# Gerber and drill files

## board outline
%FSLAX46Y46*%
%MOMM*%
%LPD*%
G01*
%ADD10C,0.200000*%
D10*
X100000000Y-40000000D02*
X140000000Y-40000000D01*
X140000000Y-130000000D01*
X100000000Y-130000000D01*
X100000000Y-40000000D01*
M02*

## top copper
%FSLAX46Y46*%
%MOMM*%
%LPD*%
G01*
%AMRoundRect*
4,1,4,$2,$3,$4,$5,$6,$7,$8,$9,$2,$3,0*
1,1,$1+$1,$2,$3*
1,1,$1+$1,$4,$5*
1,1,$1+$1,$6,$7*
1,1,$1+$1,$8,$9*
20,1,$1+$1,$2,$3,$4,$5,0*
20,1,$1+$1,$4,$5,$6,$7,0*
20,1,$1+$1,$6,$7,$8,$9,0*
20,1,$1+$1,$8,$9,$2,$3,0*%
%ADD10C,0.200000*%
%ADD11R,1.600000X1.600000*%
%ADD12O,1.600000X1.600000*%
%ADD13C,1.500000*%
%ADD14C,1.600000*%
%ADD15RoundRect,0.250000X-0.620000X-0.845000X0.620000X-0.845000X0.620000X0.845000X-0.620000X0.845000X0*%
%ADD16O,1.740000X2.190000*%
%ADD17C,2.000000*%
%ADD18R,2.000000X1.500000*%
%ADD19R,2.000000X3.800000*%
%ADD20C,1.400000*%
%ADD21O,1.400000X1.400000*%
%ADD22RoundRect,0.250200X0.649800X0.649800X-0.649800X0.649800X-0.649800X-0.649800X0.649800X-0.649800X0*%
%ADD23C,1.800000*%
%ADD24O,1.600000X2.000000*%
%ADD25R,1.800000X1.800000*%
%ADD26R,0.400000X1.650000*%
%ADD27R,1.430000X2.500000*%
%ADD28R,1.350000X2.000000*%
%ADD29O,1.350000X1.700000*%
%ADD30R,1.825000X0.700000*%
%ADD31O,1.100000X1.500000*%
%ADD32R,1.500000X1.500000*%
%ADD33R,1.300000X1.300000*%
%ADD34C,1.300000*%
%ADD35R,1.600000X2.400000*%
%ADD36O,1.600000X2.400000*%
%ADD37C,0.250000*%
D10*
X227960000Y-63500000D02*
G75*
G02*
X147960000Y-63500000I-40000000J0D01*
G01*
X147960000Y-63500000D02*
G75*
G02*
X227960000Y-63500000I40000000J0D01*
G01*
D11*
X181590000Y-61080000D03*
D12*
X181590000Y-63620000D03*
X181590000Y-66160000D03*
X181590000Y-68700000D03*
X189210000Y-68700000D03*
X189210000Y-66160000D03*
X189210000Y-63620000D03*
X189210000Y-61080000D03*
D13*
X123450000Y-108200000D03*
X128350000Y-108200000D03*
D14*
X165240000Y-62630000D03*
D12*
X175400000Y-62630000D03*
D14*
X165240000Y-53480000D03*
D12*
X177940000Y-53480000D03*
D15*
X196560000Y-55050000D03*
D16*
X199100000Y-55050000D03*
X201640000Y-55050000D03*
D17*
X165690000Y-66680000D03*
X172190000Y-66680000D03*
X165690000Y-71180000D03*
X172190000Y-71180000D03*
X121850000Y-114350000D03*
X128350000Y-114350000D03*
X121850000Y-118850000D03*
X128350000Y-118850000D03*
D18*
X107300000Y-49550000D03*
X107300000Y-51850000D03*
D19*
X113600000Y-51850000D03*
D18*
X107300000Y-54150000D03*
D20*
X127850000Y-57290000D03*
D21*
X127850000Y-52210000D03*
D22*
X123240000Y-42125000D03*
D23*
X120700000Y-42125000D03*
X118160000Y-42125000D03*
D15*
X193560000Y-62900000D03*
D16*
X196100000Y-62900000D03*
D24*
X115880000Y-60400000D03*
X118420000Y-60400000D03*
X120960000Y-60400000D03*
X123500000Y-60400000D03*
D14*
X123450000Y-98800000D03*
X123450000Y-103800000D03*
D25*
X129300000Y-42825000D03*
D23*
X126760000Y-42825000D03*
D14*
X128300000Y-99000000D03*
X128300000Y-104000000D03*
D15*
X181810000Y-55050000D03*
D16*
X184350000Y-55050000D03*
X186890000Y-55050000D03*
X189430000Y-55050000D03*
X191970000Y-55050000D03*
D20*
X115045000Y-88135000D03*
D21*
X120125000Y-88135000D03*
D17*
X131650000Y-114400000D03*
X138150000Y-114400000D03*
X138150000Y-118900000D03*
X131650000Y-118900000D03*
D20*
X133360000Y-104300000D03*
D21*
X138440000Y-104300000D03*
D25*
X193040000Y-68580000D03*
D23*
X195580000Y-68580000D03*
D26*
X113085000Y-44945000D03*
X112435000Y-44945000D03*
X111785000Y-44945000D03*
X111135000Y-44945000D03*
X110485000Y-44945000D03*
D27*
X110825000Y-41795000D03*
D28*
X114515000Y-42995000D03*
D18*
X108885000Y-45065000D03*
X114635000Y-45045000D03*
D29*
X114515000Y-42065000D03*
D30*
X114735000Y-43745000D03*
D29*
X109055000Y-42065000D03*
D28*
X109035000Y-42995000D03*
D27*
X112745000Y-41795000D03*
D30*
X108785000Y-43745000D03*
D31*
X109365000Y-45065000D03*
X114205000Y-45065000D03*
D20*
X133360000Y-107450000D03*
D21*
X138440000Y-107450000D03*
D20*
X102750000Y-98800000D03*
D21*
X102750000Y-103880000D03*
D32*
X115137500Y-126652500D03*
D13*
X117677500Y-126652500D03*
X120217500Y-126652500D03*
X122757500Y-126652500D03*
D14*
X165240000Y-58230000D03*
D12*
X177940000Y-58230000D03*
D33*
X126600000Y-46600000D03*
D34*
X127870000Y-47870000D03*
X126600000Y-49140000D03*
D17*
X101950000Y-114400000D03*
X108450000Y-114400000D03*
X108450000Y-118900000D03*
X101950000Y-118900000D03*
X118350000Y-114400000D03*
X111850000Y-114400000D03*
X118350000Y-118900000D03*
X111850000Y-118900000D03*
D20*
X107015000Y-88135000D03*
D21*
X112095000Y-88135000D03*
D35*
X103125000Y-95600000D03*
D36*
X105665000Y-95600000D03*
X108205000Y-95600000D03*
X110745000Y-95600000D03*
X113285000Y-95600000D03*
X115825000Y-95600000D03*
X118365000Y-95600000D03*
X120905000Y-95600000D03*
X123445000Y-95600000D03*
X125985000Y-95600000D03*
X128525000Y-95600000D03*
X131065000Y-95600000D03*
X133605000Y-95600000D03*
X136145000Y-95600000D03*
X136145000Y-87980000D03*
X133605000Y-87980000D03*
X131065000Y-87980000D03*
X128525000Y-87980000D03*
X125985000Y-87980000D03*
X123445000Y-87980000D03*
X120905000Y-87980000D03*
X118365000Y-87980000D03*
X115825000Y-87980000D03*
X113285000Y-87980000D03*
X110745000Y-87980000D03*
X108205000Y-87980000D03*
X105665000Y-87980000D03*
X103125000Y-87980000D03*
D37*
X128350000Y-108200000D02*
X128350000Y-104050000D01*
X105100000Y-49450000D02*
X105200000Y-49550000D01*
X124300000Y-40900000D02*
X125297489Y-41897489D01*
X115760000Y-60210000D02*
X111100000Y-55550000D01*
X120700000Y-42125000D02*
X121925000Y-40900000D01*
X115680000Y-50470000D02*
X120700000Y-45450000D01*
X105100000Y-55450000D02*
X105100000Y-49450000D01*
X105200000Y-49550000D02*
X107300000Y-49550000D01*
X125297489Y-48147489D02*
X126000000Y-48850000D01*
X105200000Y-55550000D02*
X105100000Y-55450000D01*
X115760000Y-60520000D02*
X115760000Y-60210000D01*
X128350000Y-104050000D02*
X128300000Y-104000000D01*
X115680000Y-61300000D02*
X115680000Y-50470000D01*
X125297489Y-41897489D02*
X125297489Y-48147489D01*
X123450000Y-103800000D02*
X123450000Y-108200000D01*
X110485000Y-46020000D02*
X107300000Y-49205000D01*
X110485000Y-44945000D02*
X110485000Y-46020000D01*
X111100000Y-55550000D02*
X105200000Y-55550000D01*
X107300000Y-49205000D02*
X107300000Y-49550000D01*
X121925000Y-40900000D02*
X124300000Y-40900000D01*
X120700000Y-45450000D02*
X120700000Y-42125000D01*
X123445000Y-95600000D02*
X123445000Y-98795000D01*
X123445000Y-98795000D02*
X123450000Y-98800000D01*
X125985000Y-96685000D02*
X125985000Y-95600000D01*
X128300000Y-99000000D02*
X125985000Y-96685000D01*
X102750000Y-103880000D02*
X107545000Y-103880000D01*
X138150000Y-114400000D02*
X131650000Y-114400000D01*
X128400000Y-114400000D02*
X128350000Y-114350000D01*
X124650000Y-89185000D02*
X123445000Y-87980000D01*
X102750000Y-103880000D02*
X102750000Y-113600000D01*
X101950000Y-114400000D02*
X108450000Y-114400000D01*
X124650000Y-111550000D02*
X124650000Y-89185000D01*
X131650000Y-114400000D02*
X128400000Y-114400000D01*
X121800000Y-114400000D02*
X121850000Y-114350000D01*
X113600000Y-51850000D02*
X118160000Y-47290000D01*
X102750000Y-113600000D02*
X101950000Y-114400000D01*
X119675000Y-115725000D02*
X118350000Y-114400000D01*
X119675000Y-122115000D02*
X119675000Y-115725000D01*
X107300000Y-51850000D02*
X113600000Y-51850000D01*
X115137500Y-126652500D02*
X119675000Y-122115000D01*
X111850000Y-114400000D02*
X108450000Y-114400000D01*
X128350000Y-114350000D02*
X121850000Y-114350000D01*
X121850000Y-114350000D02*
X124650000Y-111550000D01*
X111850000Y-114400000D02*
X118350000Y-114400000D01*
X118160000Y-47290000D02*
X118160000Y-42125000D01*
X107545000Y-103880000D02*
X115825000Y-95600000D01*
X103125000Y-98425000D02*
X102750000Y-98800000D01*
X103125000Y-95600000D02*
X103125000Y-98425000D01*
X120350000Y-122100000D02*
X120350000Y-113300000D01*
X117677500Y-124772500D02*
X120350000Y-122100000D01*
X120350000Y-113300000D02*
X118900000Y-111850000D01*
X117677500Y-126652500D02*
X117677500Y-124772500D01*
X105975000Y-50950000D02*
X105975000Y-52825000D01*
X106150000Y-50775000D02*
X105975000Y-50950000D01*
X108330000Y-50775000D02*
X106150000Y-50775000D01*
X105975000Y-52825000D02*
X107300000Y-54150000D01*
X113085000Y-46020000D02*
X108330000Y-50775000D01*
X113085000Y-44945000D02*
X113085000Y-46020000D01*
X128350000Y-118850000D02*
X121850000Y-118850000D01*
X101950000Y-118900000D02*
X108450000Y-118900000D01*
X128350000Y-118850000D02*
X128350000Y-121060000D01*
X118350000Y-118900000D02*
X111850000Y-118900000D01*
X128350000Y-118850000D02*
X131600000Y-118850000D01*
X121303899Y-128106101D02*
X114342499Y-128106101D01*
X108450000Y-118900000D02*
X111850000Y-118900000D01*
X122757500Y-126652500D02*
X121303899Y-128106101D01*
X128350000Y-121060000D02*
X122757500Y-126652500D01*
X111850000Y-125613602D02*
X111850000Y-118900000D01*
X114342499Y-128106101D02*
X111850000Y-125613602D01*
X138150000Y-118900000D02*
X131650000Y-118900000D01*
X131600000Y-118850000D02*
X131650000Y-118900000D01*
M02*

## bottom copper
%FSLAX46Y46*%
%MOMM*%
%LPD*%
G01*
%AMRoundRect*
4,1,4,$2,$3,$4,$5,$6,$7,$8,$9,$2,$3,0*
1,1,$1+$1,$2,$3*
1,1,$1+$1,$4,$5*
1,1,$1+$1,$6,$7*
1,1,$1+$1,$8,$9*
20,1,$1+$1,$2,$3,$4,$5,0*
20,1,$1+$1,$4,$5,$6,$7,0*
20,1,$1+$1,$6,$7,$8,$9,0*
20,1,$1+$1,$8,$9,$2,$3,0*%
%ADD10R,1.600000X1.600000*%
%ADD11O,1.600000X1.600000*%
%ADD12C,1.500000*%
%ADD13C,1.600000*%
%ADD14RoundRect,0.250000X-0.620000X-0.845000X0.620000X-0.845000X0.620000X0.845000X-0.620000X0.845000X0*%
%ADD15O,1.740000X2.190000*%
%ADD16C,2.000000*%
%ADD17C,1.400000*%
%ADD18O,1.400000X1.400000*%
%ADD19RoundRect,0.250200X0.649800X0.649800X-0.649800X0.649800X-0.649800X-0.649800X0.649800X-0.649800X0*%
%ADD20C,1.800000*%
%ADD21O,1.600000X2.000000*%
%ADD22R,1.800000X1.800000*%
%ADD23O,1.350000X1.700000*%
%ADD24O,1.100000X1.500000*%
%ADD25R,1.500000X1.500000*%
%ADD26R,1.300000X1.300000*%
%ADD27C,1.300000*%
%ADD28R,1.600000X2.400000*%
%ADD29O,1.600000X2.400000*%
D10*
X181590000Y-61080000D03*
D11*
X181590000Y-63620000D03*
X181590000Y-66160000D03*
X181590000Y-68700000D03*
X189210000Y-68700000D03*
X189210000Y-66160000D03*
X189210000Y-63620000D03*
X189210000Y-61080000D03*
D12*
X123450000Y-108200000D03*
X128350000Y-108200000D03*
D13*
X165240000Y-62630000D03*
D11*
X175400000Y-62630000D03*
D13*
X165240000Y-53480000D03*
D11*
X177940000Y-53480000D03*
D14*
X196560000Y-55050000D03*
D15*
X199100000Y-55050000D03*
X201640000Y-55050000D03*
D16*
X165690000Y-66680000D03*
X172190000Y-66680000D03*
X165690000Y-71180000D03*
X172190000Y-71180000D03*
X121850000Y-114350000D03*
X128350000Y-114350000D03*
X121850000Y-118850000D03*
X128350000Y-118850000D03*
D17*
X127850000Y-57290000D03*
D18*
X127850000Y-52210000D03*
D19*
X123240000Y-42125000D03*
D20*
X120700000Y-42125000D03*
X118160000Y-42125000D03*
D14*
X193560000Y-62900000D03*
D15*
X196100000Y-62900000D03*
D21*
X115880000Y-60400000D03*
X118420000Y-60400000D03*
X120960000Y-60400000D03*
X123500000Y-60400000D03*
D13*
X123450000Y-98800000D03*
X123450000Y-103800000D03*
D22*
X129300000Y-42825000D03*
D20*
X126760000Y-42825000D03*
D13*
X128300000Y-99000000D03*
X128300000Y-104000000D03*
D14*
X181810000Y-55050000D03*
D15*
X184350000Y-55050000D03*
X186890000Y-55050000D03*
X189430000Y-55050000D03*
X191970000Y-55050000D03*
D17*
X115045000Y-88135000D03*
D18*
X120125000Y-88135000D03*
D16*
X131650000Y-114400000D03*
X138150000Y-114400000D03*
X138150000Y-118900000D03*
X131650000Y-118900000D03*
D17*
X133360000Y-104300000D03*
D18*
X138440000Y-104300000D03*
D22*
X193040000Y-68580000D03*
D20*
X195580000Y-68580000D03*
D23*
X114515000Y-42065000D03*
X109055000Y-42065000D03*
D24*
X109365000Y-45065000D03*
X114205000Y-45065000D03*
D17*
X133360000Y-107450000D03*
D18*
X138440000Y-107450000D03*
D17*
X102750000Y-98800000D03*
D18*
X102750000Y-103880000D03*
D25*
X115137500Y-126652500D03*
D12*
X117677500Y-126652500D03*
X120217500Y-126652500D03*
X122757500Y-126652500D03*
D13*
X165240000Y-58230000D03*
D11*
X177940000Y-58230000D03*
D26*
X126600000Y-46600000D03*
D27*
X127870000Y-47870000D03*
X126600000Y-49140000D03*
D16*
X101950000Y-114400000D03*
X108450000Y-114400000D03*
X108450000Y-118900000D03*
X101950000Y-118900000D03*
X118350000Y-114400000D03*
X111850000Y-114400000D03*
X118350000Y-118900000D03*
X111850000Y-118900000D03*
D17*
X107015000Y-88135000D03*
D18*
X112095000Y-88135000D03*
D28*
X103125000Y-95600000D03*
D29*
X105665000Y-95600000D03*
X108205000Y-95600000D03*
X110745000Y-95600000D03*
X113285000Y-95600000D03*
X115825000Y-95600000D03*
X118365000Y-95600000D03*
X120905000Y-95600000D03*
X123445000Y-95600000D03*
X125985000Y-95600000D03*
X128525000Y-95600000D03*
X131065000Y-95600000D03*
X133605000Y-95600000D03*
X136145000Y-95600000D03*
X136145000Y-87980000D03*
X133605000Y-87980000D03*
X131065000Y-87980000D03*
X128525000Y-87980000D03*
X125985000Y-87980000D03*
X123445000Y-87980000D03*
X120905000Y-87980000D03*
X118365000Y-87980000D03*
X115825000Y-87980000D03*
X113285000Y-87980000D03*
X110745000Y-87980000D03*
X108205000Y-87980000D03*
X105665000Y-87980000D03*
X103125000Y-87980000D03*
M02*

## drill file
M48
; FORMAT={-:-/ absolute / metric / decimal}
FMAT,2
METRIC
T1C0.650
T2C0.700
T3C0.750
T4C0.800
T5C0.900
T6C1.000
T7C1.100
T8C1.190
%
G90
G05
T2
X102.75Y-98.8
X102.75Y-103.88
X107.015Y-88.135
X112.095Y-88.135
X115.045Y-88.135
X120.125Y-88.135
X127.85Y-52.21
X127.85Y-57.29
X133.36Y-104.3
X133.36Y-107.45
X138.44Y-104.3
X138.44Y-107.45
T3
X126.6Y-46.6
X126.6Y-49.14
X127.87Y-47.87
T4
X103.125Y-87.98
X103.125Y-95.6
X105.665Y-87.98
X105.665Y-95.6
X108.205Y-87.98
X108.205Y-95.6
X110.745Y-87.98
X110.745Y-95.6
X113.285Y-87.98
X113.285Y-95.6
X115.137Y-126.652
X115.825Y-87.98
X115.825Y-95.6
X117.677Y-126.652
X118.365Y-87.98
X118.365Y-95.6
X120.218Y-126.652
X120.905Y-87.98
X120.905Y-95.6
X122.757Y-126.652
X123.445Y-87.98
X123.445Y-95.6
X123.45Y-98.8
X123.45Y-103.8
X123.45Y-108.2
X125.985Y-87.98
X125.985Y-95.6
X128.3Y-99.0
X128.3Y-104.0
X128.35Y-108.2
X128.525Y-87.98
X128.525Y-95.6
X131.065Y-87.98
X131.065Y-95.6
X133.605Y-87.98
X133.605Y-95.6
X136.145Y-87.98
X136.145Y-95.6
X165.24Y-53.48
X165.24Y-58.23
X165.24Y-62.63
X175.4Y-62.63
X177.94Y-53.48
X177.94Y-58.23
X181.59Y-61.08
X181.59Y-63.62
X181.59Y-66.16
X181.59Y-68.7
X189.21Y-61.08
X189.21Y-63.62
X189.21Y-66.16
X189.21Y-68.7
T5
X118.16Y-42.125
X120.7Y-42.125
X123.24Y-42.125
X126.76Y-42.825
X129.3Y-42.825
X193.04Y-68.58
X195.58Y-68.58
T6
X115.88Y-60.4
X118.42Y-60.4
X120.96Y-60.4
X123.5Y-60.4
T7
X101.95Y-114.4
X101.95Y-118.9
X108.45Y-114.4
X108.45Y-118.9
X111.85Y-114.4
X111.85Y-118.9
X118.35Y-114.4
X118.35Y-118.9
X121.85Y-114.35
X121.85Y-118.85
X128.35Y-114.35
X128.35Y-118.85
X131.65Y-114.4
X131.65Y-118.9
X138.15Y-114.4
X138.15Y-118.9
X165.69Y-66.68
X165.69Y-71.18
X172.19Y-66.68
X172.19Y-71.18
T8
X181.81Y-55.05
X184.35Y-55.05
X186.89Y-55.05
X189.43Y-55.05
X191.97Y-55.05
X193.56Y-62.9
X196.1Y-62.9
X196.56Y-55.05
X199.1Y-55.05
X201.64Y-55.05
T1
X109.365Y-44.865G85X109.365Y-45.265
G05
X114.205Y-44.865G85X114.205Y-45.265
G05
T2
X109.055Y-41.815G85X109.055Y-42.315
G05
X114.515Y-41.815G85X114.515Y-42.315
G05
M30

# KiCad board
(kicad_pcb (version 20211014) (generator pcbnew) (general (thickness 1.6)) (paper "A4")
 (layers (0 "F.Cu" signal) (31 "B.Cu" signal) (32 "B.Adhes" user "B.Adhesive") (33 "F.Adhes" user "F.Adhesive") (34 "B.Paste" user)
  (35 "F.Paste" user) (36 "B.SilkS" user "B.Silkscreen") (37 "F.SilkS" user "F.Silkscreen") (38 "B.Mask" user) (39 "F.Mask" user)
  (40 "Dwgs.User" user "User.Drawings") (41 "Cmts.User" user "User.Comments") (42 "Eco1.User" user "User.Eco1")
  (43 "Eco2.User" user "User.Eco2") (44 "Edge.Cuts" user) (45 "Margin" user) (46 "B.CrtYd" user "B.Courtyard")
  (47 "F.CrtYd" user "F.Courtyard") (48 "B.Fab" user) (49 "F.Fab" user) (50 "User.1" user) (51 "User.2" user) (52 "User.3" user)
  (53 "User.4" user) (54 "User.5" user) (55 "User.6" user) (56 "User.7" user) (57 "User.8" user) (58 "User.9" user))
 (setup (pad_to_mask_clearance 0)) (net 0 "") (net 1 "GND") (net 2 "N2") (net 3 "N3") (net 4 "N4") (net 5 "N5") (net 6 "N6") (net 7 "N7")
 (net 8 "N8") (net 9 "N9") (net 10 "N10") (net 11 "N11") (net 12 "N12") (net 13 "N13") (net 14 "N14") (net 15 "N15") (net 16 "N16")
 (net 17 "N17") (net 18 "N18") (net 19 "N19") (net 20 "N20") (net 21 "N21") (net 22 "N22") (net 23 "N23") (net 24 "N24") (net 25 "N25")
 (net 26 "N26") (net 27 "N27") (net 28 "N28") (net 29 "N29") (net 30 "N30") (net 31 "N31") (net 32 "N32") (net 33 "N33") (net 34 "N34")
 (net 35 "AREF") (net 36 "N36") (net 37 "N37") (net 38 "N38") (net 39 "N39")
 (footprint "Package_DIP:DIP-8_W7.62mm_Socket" (layer "F.Cu") (at 181.59 61.08)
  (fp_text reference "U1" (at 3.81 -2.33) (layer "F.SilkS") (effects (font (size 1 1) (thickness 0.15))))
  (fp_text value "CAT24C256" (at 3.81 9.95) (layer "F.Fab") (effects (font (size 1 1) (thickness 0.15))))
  (pad "1" thru_hole rect (at 0 0) (size 1.6 1.6) (drill 0.8) (layers *.Cu *.Mask) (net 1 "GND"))
  (pad "2" thru_hole oval (at 0 2.54) (size 1.6 1.6) (drill 0.8) (layers *.Cu *.Mask) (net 1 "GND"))
  (pad "3" thru_hole oval (at 0 5.08) (size 1.6 1.6) (drill 0.8) (layers *.Cu *.Mask) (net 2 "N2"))
  (pad "4" thru_hole oval (at 0 7.62) (size 1.6 1.6) (drill 0.8) (layers *.Cu *.Mask) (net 1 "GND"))
  (pad "5" thru_hole oval (at 7.62 7.62) (size 1.6 1.6) (drill 0.8) (layers *.Cu *.Mask) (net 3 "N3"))
  (pad "6" thru_hole oval (at 7.62 5.08) (size 1.6 1.6) (drill 0.8) (layers *.Cu *.Mask) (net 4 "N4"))
  (pad "7" thru_hole oval (at 7.62 2.54) (size 1.6 1.6) (drill 0.8) (layers *.Cu *.Mask) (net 1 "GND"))
  (pad "8" thru_hole oval (at 7.62 0) (size 1.6 1.6) (drill 0.8) (layers *.Cu *.Mask) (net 2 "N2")))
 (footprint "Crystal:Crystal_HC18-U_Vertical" (layer "F.Cu") (at 123.45 108.2)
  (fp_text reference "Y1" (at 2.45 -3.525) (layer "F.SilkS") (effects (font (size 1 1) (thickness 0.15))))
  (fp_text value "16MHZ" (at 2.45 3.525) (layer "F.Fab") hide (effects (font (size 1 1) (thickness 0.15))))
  (pad "1" thru_hole circle (at 0 0) (size 1.5 1.5) (drill 0.8) (layers *.Cu *.Mask) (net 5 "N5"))
  (pad "2" thru_hole circle (at 4.9 0) (size 1.5 1.5) (drill 0.8) (layers *.Cu *.Mask) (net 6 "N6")))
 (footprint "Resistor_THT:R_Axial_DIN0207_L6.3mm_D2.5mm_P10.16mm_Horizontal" (layer "F.Cu") (at 165.24 62.63)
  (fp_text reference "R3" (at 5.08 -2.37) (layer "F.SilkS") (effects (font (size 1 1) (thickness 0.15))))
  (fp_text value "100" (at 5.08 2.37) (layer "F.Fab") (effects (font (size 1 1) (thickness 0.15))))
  (pad "1" thru_hole circle (at 0 0) (size 1.6 1.6) (drill 0.8) (layers *.Cu *.Mask) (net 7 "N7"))
  (pad "2" thru_hole oval (at 10.16 0) (size 1.6 1.6) (drill 0.8) (layers *.Cu *.Mask) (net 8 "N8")))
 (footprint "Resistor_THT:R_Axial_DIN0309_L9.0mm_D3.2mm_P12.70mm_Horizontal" (layer "F.Cu") (at 165.24 53.48)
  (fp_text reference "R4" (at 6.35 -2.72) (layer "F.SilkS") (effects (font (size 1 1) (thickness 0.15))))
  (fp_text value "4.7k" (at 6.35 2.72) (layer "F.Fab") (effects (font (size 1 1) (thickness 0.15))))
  (pad "1" thru_hole circle (at 0 0) (size 1.6 1.6) (drill 0.8) (layers *.Cu *.Mask) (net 3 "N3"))
  (pad "2" thru_hole oval (at 12.7 0) (size 1.6 1.6) (drill 0.8) (layers *.Cu *.Mask) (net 2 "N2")))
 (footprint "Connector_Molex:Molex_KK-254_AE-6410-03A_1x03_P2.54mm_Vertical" (layer "F.Cu") (at 196.56 55.05)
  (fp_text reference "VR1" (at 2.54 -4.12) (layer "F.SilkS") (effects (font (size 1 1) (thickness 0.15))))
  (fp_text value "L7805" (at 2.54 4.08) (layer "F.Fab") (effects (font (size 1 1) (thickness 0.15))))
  (pad "1" thru_hole roundrect (at 0 0) (size 1.74 2.19) (drill 1.19) (layers *.Cu *.Mask) (roundrect_rratio 0.143678) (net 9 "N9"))
  (pad "2" thru_hole oval (at 2.54 0) (size 1.74 2.19) (drill 1.19) (layers *.Cu *.Mask) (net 1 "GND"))
  (pad "3" thru_hole oval (at 5.08 0) (size 1.74 2.19) (drill 1.19) (layers *.Cu *.Mask) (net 2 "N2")))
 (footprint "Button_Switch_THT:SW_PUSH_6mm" (layer "F.Cu") (at 165.69 66.68)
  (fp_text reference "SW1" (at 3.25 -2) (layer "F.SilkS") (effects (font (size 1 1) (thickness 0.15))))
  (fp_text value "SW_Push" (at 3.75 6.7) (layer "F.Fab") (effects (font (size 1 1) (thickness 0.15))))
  (pad "1" thru_hole circle (at 0 0 90) (size 2 2) (drill 1.1) (layers *.Cu *.Mask) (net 1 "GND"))
  (pad "1" thru_hole circle (at 6.5 0 90) (size 2 2) (drill 1.1) (layers *.Cu *.Mask) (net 1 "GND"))
  (pad "2" thru_hole circle (at 0 4.5 90) (size 2 2) (drill 1.1) (layers *.Cu *.Mask) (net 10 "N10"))
  (pad "2" thru_hole circle (at 6.5 4.5 90) (size 2 2) (drill 1.1) (layers *.Cu *.Mask) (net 10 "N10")))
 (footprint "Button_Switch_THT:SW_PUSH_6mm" (layer "F.Cu") (at 121.85 114.35)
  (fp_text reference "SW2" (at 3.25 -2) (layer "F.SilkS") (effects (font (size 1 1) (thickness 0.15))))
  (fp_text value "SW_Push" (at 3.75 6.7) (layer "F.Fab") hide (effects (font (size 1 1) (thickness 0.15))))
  (pad "1" thru_hole circle (at 0 0 90) (size 2 2) (drill 1.1) (layers *.Cu *.Mask) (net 2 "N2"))
  (pad "1" thru_hole circle (at 6.5 0 90) (size 2 2) (drill 1.1) (layers *.Cu *.Mask) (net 2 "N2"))
  (pad "2" thru_hole circle (at 0 4.5 90) (size 2 2) (drill 1.1) (layers *.Cu *.Mask) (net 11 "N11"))
  (pad "2" thru_hole circle (at 6.5 4.5 90) (size 2 2) (drill 1.1) (layers *.Cu *.Mask) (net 11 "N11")))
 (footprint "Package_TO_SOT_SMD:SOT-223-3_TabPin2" (layer "F.Cu") (at 110.45 51.85)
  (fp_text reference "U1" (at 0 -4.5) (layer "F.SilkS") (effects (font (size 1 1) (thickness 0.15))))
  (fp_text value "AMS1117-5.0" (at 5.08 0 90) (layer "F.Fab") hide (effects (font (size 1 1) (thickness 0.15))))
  (pad "1" smd rect (at -3.15 -2.3) (size 2 1.5) (layers "F.Cu" "F.Paste" "F.Mask") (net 1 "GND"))
  (pad "2" smd rect (at -3.15 0) (size 2 1.5) (layers "F.Cu" "F.Paste" "F.Mask") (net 2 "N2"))
  (pad "2" smd rect (at 3.15 0) (size 2 3.8) (layers "F.Cu" "F.Paste" "F.Mask") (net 2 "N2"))
  (pad "3" smd rect (at -3.15 2.3) (size 2 1.5) (layers "F.Cu" "F.Paste" "F.Mask") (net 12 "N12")))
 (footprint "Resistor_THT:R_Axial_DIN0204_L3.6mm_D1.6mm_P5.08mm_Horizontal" (layer "F.Cu") (at 127.85 57.29 90)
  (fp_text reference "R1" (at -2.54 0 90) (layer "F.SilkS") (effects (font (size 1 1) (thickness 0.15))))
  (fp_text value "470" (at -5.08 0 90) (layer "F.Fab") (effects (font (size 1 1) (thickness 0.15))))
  (pad "1" thru_hole circle (at 0 0 90) (size 1.4 1.4) (drill 0.7) (layers *.Cu *.Mask) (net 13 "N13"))
  (pad "2" thru_hole oval (at 5.08 0 90) (size 1.4 1.4) (drill 0.7) (layers *.Cu *.Mask) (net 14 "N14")))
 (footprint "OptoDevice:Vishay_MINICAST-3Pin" (layer "F.Cu") (at 123.24 42.125 180)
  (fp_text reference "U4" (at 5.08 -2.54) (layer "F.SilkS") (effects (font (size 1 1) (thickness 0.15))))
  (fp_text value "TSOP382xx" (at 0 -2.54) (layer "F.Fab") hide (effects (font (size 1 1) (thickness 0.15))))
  (pad "1" thru_hole roundrect (at 0 0 180) (size 1.8 1.8) (drill 0.9) (layers *.Cu *.Mask) (roundrect_rratio 0.139) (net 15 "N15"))
  (pad "2" thru_hole circle (at 2.54 0 180) (size 1.8 1.8) (drill 0.9) (layers *.Cu *.Mask) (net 1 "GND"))
  (pad "3" thru_hole circle (at 5.08 0 180) (size 1.8 1.8) (drill 0.9) (layers *.Cu *.Mask) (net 2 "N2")))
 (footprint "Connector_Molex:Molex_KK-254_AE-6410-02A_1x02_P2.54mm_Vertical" (layer "F.Cu") (at 193.56 62.9)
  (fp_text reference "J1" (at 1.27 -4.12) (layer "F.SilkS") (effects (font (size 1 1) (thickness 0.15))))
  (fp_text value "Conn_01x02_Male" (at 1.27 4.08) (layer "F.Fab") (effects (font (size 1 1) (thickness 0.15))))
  (pad "1" thru_hole roundrect (at 0 0) (size 1.74 2.19) (drill 1.19) (layers *.Cu *.Mask) (roundrect_rratio 0.143678) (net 9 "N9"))
  (pad "2" thru_hole oval (at 2.54 0) (size 1.74 2.19) (drill 1.19) (layers *.Cu *.Mask) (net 1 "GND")))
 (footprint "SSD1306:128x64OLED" (layer "F.Cu") (at 119.5 71)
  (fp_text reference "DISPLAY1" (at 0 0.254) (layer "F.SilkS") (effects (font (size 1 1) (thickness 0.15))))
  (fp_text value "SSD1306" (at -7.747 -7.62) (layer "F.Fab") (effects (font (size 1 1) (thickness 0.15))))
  (pad "1" thru_hole oval locked (at -3.62 -10.6 90) (size 2 1.6) (drill 1) (layers *.Cu *.Mask) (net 1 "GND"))
  (pad "2" thru_hole oval locked (at -1.08 -10.6 90) (size 2 1.6) (drill 1) (layers *.Cu *.Mask) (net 2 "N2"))
  (pad "3" thru_hole oval locked (at 1.46 -10.6 90) (size 2 1.6) (drill 1) (layers *.Cu *.Mask) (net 4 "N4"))
  (pad "4" thru_hole oval locked (at 4 -10.6 90) (size 2 1.6) (drill 1) (layers *.Cu *.Mask) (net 3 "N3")))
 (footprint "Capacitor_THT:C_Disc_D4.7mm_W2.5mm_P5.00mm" (layer "F.Cu") (at 123.45 98.8 -90)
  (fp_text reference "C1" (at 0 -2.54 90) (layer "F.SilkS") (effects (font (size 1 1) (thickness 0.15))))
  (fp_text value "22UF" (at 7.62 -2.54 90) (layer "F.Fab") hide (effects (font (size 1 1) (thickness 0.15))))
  (pad "1" thru_hole circle (at 0 0 270) (size 1.6 1.6) (drill 0.8) (layers *.Cu *.Mask) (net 5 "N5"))
  (pad "2" thru_hole circle (at 5 0 270) (size 1.6 1.6) (drill 0.8) (layers *.Cu *.Mask) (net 1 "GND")))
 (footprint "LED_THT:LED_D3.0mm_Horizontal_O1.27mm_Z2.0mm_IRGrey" (layer "F.Cu") (at 129.3 42.825 180)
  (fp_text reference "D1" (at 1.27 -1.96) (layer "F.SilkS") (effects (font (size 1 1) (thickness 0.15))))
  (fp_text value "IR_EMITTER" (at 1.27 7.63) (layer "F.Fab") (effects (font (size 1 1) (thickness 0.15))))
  (pad "1" thru_hole rect (at 0 0 180) (size 1.8 1.8) (drill 0.9) (layers *.Cu *.Mask))
  (pad "2" thru_hole circle (at 2.54 0 180) (size 1.8 1.8) (drill 0.9) (layers *.Cu *.Mask)))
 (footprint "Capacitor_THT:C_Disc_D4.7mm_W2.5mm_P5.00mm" (layer "F.Cu") (at 128.3 99 -90)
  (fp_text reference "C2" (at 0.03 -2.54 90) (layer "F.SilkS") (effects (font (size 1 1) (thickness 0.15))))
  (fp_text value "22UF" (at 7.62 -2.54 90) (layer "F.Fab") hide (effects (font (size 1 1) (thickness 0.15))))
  (pad "1" thru_hole circle (at 0 0 270) (size 1.6 1.6) (drill 0.8) (layers *.Cu *.Mask) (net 6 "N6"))
  (pad "2" thru_hole circle (at 5 0 270) (size 1.6 1.6) (drill 0.8) (layers *.Cu *.Mask) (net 1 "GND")))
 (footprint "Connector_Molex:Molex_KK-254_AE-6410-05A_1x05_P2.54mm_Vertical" (layer "F.Cu") (at 181.81 55.05)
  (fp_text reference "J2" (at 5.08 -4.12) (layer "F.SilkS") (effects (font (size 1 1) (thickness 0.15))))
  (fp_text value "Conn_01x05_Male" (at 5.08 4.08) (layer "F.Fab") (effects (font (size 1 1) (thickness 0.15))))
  (pad "1" thru_hole roundrect (at 0 0) (size 1.74 2.19) (drill 1.19) (layers *.Cu *.Mask) (roundrect_rratio 0.143678) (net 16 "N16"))
  (pad "2" thru_hole oval (at 2.54 0) (size 1.74 2.19) (drill 1.19) (layers *.Cu *.Mask) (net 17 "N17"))
  (pad "3" thru_hole oval (at 5.08 0) (size 1.74 2.19) (drill 1.19) (layers *.Cu *.Mask) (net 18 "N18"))
  (pad "4" thru_hole oval (at 7.62 0) (size 1.74 2.19) (drill 1.19) (layers *.Cu *.Mask) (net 2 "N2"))
  (pad "5" thru_hole oval (at 10.16 0) (size 1.74 2.19) (drill 1.19) (layers *.Cu *.Mask) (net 1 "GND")))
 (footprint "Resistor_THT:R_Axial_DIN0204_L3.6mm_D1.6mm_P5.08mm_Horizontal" (layer "F.Cu") (at 115.045 88.135)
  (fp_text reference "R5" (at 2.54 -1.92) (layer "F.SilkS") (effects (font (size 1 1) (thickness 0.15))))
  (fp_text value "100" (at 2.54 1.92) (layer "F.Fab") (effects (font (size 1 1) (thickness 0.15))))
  (pad "1" thru_hole circle (at 0 0) (size 1.4 1.4) (drill 0.7) (layers *.Cu *.Mask) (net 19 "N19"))
  (pad "2" thru_hole oval (at 5.08 0) (size 1.4 1.4) (drill 0.7) (layers *.Cu *.Mask) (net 1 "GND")))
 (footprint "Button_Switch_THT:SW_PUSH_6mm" (layer "F.Cu") (at 131.65 114.4)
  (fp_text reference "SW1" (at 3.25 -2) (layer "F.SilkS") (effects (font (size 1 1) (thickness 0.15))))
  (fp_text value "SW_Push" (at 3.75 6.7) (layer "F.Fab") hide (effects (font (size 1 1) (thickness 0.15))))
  (pad "1" thru_hole circle (at 0 0 90) (size 2 2) (drill 1.1) (layers *.Cu *.Mask) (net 2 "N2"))
  (pad "1" thru_hole circle (at 6.5 0 90) (size 2 2) (drill 1.1) (layers *.Cu *.Mask) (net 2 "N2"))
  (pad "2" thru_hole circle (at 6.5 4.5 90) (size 2 2) (drill 1.1) (layers *.Cu *.Mask) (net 7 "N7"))
  (pad "2" thru_hole circle (at 0 4.5 90) (size 2 2) (drill 1.1) (layers *.Cu *.Mask) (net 7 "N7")))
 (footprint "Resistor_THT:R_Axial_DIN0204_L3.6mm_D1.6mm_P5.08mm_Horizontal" (layer "F.Cu") (at 133.36 104.3)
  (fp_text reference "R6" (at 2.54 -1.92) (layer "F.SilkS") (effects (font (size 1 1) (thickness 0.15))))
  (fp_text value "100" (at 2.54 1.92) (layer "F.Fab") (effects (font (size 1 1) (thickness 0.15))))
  (pad "1" thru_hole circle (at 0 0) (size 1.4 1.4) (drill 0.7) (layers *.Cu *.Mask) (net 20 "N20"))
  (pad "2" thru_hole oval (at 5.08 0) (size 1.4 1.4) (drill 0.7) (layers *.Cu *.Mask) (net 1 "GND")))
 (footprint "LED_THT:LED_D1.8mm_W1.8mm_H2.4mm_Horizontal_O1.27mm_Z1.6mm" (layer "F.Cu") (at 193.04 68.58)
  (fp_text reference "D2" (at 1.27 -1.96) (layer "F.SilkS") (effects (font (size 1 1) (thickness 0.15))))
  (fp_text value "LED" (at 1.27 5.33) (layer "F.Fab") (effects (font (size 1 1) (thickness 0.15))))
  (pad "1" thru_hole rect (at 0 0) (size 1.8 1.8) (drill 0.9) (layers *.Cu *.Mask) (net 7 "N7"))
  (pad "2" thru_hole circle (at 2.54 0) (size 1.8 1.8) (drill 0.9) (layers *.Cu *.Mask) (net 2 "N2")))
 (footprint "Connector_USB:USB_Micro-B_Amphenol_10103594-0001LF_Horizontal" (layer "F.Cu") (at 111.76 43.18 180)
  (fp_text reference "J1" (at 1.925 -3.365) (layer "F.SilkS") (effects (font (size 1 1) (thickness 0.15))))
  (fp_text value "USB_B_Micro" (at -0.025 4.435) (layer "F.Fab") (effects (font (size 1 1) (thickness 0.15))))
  (pad "1" smd rect (at -1.325 -1.765 270) (size 1.65 0.4) (layers "F.Cu" "F.Paste" "F.Mask") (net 12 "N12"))
  (pad "2" smd rect (at -0.675 -1.765 270) (size 1.65 0.4) (layers "F.Cu" "F.Paste" "F.Mask") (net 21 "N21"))
  (pad "3" smd rect (at -0.025 -1.765 270) (size 1.65 0.4) (layers "F.Cu" "F.Paste" "F.Mask") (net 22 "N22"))
  (pad "4" smd rect (at 0.625 -1.765 270) (size 1.65 0.4) (layers "F.Cu" "F.Paste" "F.Mask") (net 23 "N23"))
  (pad "5" smd rect (at 1.275 -1.765 270) (size 1.65 0.4) (layers "F.Cu" "F.Paste" "F.Mask") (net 1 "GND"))
  (pad "6" smd rect (at 0.935 1.385 270) (size 2.5 1.43) (layers "F.Cu" "F.Paste" "F.Mask") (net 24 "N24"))
  (pad "6" smd rect (at -2.755 0.185 180) (size 1.35 2) (layers "F.Cu" "F.Paste" "F.Mask") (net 24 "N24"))
  (pad "6" smd rect (at 2.875 -1.885 180) (size 2 1.5) (layers "F.Cu" "F.Paste" "F.Mask") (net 24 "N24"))
  (pad "6" smd rect (at -2.875 -1.865 180) (size 2 1.5) (layers "F.Cu" "F.Paste" "F.Mask") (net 24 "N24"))
  (pad "6" thru_hole oval (at -2.755 1.115 270) (size 1.7 1.35) (drill oval 1.2 0.7) (layers *.Cu *.Mask) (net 24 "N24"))
  (pad "6" smd rect (at -2.975 -0.565 180) (size 1.825 0.7) (layers "F.Cu" "F.Paste" "F.Mask") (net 24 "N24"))
  (pad "6" thru_hole oval (at 2.705 1.115 270) (size 1.7 1.35) (drill oval 1.2 0.7) (layers *.Cu *.Mask) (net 24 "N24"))
  (pad "6" smd rect (at 2.725 0.185 180) (size 1.35 2) (layers "F.Cu" "F.Paste" "F.Mask") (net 24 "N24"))
  (pad "6" smd rect (at -0.985 1.385 270) (size 2.5 1.43) (layers "F.Cu" "F.Paste" "F.Mask") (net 24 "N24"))
  (pad "6" smd rect (at 2.975 -0.565 180) (size 1.825 0.7) (layers "F.Cu" "F.Paste" "F.Mask") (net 24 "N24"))
  (pad "6" thru_hole oval (at 2.395 -1.885 270) (size 1.5 1.1) (drill oval 1.05 0.65) (layers *.Cu *.Mask) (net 24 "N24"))
  (pad "6" thru_hole oval (at -2.445 -1.885 270) (size 1.5 1.1) (drill oval 1.05 0.65) (layers *.Cu *.Mask) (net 24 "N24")))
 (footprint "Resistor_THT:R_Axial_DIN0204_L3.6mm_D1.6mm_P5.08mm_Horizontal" (layer "F.Cu") (at 133.36 107.45)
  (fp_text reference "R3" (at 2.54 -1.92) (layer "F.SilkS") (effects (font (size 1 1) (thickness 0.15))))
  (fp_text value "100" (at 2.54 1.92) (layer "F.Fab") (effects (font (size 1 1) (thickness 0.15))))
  (pad "1" thru_hole circle (at 0 0) (size 1.4 1.4) (drill 0.7) (layers *.Cu *.Mask) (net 7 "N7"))
  (pad "2" thru_hole oval (at 5.08 0) (size 1.4 1.4) (drill 0.7) (layers *.Cu *.Mask) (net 1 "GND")))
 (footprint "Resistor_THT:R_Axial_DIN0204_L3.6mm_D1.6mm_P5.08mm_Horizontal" (layer "F.Cu") (at 102.75 98.8 -90)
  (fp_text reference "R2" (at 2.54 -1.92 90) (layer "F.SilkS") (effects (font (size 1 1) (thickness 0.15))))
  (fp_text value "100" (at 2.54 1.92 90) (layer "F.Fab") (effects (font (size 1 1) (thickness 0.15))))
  (pad "1" thru_hole circle (at 0 0 270) (size 1.4 1.4) (drill 0.7) (layers *.Cu *.Mask) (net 10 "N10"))
  (pad "2" thru_hole oval (at 5.08 0 270) (size 1.4 1.4) (drill 0.7) (layers *.Cu *.Mask) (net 2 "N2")))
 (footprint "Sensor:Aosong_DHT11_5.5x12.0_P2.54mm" (layer "F.Cu") (at 115.1375 126.6525 90)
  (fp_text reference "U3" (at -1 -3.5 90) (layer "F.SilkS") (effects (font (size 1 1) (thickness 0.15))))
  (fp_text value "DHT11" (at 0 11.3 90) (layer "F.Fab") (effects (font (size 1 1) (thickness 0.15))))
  (pad "1" thru_hole rect (at 0 0 90) (size 1.5 1.5) (drill 0.8) (layers *.Cu *.Mask) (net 2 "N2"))
  (pad "2" thru_hole circle (at 0 2.54 90) (size 1.5 1.5) (drill 0.8) (layers *.Cu *.Mask) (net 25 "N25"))
  (pad "3" thru_hole circle (at 0 5.08 90) (size 1.5 1.5) (drill 0.8) (layers *.Cu *.Mask) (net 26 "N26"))
  (pad "4" thru_hole circle (at 0 7.62 90) (size 1.5 1.5) (drill 0.8) (layers *.Cu *.Mask) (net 1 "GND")))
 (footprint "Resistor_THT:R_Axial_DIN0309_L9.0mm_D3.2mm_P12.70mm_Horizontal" (layer "F.Cu") (at 165.24 58.23)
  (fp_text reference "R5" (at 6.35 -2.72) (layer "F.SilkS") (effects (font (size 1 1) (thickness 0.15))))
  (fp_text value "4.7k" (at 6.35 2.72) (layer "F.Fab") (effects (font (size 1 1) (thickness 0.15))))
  (pad "1" thru_hole circle (at 0 0) (size 1.6 1.6) (drill 0.8) (layers *.Cu *.Mask) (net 4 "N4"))
  (pad "2" thru_hole oval (at 12.7 0) (size 1.6 1.6) (drill 0.8) (layers *.Cu *.Mask) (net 2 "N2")))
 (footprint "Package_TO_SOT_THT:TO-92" (layer "F.Cu") (at 126.6 46.6 -90)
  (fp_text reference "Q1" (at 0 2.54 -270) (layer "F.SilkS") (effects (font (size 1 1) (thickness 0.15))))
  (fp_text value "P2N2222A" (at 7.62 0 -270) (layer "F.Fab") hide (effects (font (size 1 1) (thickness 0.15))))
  (pad "1" thru_hole rect (at 0 0 270) (size 1.3 1.3) (drill 0.75) (layers *.Cu *.Mask) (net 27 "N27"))
  (pad "2" thru_hole circle (at 1.27 -1.27 270) (size 1.3 1.3) (drill 0.75) (layers *.Cu *.Mask) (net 14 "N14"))
  (pad "3" thru_hole circle (at 2.54 0 270) (size 1.3 1.3) (drill 0.75) (layers *.Cu *.Mask) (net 1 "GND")))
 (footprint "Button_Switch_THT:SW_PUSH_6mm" (layer "F.Cu") (at 101.95 114.4)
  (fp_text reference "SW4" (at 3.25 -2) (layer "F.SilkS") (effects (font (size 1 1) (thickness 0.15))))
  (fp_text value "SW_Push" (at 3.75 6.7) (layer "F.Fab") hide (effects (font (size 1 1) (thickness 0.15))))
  (pad "1" thru_hole circle (at 0 0 90) (size 2 2) (drill 1.1) (layers *.Cu *.Mask) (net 2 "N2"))
  (pad "1" thru_hole circle (at 6.5 0 90) (size 2 2) (drill 1.1) (layers *.Cu *.Mask) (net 2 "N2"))
  (pad "2" thru_hole circle (at 6.5 4.5 90) (size 2 2) (drill 1.1) (layers *.Cu *.Mask) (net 20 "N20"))
  (pad "2" thru_hole circle (at 0 4.5 90) (size 2 2) (drill 1.1) (layers *.Cu *.Mask) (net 20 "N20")))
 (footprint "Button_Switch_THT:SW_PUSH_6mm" (layer "F.Cu") (at 111.85 114.4)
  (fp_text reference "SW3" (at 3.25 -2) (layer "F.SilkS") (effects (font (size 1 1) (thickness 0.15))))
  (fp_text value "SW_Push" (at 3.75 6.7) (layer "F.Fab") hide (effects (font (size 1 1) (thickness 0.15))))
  (pad "1" thru_hole circle (at 6.5 0 90) (size 2 2) (drill 1.1) (layers *.Cu *.Mask) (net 2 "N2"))
  (pad "1" thru_hole circle (at 0 0 90) (size 2 2) (drill 1.1) (layers *.Cu *.Mask) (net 2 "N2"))
  (pad "2" thru_hole circle (at 6.5 4.5 90) (size 2 2) (drill 1.1) (layers *.Cu *.Mask) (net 19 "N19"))
  (pad "2" thru_hole circle (at 0 4.5 90) (size 2 2) (drill 1.1) (layers *.Cu *.Mask) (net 19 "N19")))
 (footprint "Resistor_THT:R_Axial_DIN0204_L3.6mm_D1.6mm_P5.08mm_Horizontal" (layer "F.Cu") (at 107.015 88.135)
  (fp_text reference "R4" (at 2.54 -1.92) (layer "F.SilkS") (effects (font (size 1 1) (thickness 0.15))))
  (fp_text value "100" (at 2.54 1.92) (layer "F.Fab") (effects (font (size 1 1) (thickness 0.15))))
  (pad "1" thru_hole circle (at 0 0) (size 1.4 1.4) (drill 0.7) (layers *.Cu *.Mask) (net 11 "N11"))
  (pad "2" thru_hole oval (at 5.08 0) (size 1.4 1.4) (drill 0.7) (layers *.Cu *.Mask) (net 1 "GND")))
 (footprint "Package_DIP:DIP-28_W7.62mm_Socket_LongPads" (layer "F.Cu") (at 103.125 95.6 90)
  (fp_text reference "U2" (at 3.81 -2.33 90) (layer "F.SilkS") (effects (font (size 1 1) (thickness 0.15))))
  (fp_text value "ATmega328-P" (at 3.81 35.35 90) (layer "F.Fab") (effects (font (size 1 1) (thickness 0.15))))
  (pad "1" thru_hole rect (at 0 0 90) (size 2.4 1.6) (drill 0.8) (layers *.Cu *.Mask) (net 10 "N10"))
  (pad "2" thru_hole oval (at 0 2.54 90) (size 2.4 1.6) (drill 0.8) (layers *.Cu *.Mask) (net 25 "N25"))
  (pad "3" thru_hole oval (at 0 5.08 90) (size 2.4 1.6) (drill 0.8) (layers *.Cu *.Mask) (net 13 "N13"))
  (pad "4" thru_hole oval (at 0 7.62 90) (size 2.4 1.6) (drill 0.8) (layers *.Cu *.Mask) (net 15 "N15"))
  (pad "5" thru_hole oval (at 0 10.16 90) (size 2.4 1.6) (drill 0.8) (layers *.Cu *.Mask) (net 18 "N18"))
  (pad "6" thru_hole oval (at 0 12.7 90) (size 2.4 1.6) (drill 0.8) (layers *.Cu *.Mask) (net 17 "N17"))
  (pad "7" thru_hole oval (at 0 15.24 90) (size 2.4 1.6) (drill 0.8) (layers *.Cu *.Mask) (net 2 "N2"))
  (pad "8" thru_hole oval (at 0 17.78 90) (size 2.4 1.6) (drill 0.8) (layers *.Cu *.Mask) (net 1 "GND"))
  (pad "9" thru_hole oval (at 0 20.32 90) (size 2.4 1.6) (drill 0.8) (layers *.Cu *.Mask) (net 5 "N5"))
  (pad "10" thru_hole oval (at 0 22.86 90) (size 2.4 1.6) (drill 0.8) (layers *.Cu *.Mask) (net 6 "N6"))
  (pad "11" thru_hole oval (at 0 25.4 90) (size 2.4 1.6) (drill 0.8) (layers *.Cu *.Mask) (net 16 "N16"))
  (pad "12" thru_hole oval (at 0 27.94 90) (size 2.4 1.6) (drill 0.8) (layers *.Cu *.Mask) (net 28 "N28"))
  (pad "13" thru_hole oval (at 0 30.48 90) (size 2.4 1.6) (drill 0.8) (layers *.Cu *.Mask) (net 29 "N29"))
  (pad "14" thru_hole oval (at 0 33.02 90) (size 2.4 1.6) (drill 0.8) (layers *.Cu *.Mask) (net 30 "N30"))
  (pad "15" thru_hole oval (at 7.62 33.02 90) (size 2.4 1.6) (drill 0.8) (layers *.Cu *.Mask) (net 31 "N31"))
  (pad "16" thru_hole oval (at 7.62 30.48 90) (size 2.4 1.6) (drill 0.8) (layers *.Cu *.Mask) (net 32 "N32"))
  (pad "17" thru_hole oval (at 7.62 27.94 90) (size 2.4 1.6) (drill 0.8) (layers *.Cu *.Mask) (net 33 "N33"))
  (pad "18" thru_hole oval (at 7.62 25.4 90) (size 2.4 1.6) (drill 0.8) (layers *.Cu *.Mask) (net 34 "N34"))
  (pad "19" thru_hole oval (at 7.62 22.86 90) (size 2.4 1.6) (drill 0.8) (layers *.Cu *.Mask) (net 8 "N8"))
  (pad "20" thru_hole oval (at 7.62 20.32 90) (size 2.4 1.6) (drill 0.8) (layers *.Cu *.Mask) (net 2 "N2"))
  (pad "21" thru_hole oval (at 7.62 17.78 90) (size 2.4 1.6) (drill 0.8) (layers *.Cu *.Mask) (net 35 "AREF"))
  (pad "22" thru_hole oval (at 7.62 15.24 90) (size 2.4 1.6) (drill 0.8) (layers *.Cu *.Mask) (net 1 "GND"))
  (pad "23" thru_hole oval (at 7.62 12.7 90) (size 2.4 1.6) (drill 0.8) (layers *.Cu *.Mask) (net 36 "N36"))
  (pad "24" thru_hole oval (at 7.62 10.16 90) (size 2.4 1.6) (drill 0.8) (layers *.Cu *.Mask) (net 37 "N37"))
  (pad "25" thru_hole oval (at 7.62 7.62 90) (size 2.4 1.6) (drill 0.8) (layers *.Cu *.Mask) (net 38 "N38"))
  (pad "26" thru_hole oval (at 7.62 5.08 90) (size 2.4 1.6) (drill 0.8) (layers *.Cu *.Mask) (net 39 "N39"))
  (pad "27" thru_hole oval (at 7.62 2.54 90) (size 2.4 1.6) (drill 0.8) (layers *.Cu *.Mask) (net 3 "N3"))
  (pad "28" thru_hole oval (at 7.62 0 90) (size 2.4 1.6) (drill 0.8) (layers *.Cu *.Mask) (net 4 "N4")))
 (gr_circle (center 187.96 63.5) (end 227.96 63.5) (layer "F.Cu") (width 0.2) (fill none))
 (gr_rect (start 100 40) (end 140 130) (layer "Edge.Cuts") (width 0.2) (fill none))
 (segment (start 128.35 108.2) (end 128.35 104.05) (width 0.25) (layer "F.Cu") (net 1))
 (segment (start 105.1 49.45) (end 105.2 49.55) (width 0.25) (layer "F.Cu") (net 1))
 (segment (start 124.3 40.9) (end 125.297489 41.897489) (width 0.25) (layer "F.Cu") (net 1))
 (segment (start 115.76 60.21) (end 111.1 55.55) (width 0.25) (layer "F.Cu") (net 1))
 (segment (start 120.7 42.125) (end 121.925 40.9) (width 0.25) (layer "F.Cu") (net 1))
 (segment (start 115.68 50.47) (end 120.7 45.45) (width 0.25) (layer "F.Cu") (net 1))
 (segment (start 105.1 55.45) (end 105.1 49.45) (width 0.25) (layer "F.Cu") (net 1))
 (segment (start 105.2 49.55) (end 107.3 49.55) (width 0.25) (layer "F.Cu") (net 1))
 (segment (start 125.297489 48.147489) (end 126 48.85) (width 0.25) (layer "F.Cu") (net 1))
 (segment (start 105.2 55.55) (end 105.1 55.45) (width 0.25) (layer "F.Cu") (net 1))
 (segment (start 115.76 60.52) (end 115.76 60.21) (width 0.25) (layer "F.Cu") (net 1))
 (segment (start 128.35 104.05) (end 128.3 104) (width 0.25) (layer "F.Cu") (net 1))
 (segment (start 115.68 61.3) (end 115.68 50.47) (width 0.25) (layer "F.Cu") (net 1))
 (segment (start 125.297489 41.897489) (end 125.297489 48.147489) (width 0.25) (layer "F.Cu") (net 1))
 (segment (start 123.45 103.8) (end 123.45 108.2) (width 0.25) (layer "F.Cu") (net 1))
 (segment (start 110.485 46.02) (end 107.3 49.205) (width 0.25) (layer "F.Cu") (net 1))
 (segment (start 110.485 44.945) (end 110.485 46.02) (width 0.25) (layer "F.Cu") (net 1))
 (segment (start 111.1 55.55) (end 105.2 55.55) (width 0.25) (layer "F.Cu") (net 1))
 (segment (start 107.3 49.205) (end 107.3 49.55) (width 0.25) (layer "F.Cu") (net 1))
 (segment (start 121.925 40.9) (end 124.3 40.9) (width 0.25) (layer "F.Cu") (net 1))
 (segment (start 120.7 45.45) (end 120.7 42.125) (width 0.25) (layer "F.Cu") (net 1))
 (segment (start 123.445 95.6) (end 123.445 98.795) (width 0.25) (layer "F.Cu") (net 5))
 (segment (start 123.445 98.795) (end 123.45 98.8) (width 0.25) (layer "F.Cu") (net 5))
 (segment (start 125.985 96.685) (end 125.985 95.6) (width 0.25) (layer "F.Cu") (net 6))
 (segment (start 128.3 99) (end 125.985 96.685) (width 0.25) (layer "F.Cu") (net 6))
 (segment (start 102.75 103.88) (end 107.545 103.88) (width 0.25) (layer "F.Cu") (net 2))
 (segment (start 138.15 114.4) (end 131.65 114.4) (width 0.25) (layer "F.Cu") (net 2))
 (segment (start 128.4 114.4) (end 128.35 114.35) (width 0.25) (layer "F.Cu") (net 2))
 (segment (start 124.65 89.185) (end 123.445 87.98) (width 0.25) (layer "F.Cu") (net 2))
 (segment (start 102.75 103.88) (end 102.75 113.6) (width 0.25) (layer "F.Cu") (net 2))
 (segment (start 101.95 114.4) (end 108.45 114.4) (width 0.25) (layer "F.Cu") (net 2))
 (segment (start 124.65 111.55) (end 124.65 89.185) (width 0.25) (layer "F.Cu") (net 2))
 (segment (start 131.65 114.4) (end 128.4 114.4) (width 0.25) (layer "F.Cu") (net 2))
 (segment (start 121.8 114.4) (end 121.85 114.35) (width 0.25) (layer "F.Cu") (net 2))
 (segment (start 113.6 51.85) (end 118.16 47.29) (width 0.25) (layer "F.Cu") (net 2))
 (segment (start 102.75 113.6) (end 101.95 114.4) (width 0.25) (layer "F.Cu") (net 2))
 (segment (start 119.675 115.725) (end 118.35 114.4) (width 0.25) (layer "F.Cu") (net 2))
 (segment (start 119.675 122.115) (end 119.675 115.725) (width 0.25) (layer "F.Cu") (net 2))
 (segment (start 107.3 51.85) (end 113.6 51.85) (width 0.25) (layer "F.Cu") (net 2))
 (segment (start 115.1375 126.6525) (end 119.675 122.115) (width 0.25) (layer "F.Cu") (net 2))
 (segment (start 111.85 114.4) (end 108.45 114.4) (width 0.25) (layer "F.Cu") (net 2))
 (segment (start 128.35 114.35) (end 121.85 114.35) (width 0.25) (layer "F.Cu") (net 2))
 (segment (start 121.85 114.35) (end 124.65 111.55) (width 0.25) (layer "F.Cu") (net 2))
 (segment (start 111.85 114.4) (end 118.35 114.4) (width 0.25) (layer "F.Cu") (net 2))
 (segment (start 118.16 47.29) (end 118.16 42.125) (width 0.25) (layer "F.Cu") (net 2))
 (segment (start 107.545 103.88) (end 115.825 95.6) (width 0.25) (layer "F.Cu") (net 2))
 (segment (start 103.125 98.425) (end 102.75 98.8) (width 0.25) (layer "F.Cu") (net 10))
 (segment (start 103.125 95.6) (end 103.125 98.425) (width 0.25) (layer "F.Cu") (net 10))
 (segment (start 120.35 122.1) (end 120.35 113.3) (width 0.25) (layer "F.Cu") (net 25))
 (segment (start 117.6775 124.7725) (end 120.35 122.1) (width 0.25) (layer "F.Cu") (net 25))
 (segment (start 120.35 113.3) (end 118.9 111.85) (width 0.25) (layer "F.Cu") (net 25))
 (segment (start 117.6775 126.6525) (end 117.6775 124.7725) (width 0.25) (layer "F.Cu") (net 25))
 (segment (start 105.975 50.95) (end 105.975 52.825) (width 0.25) (layer "F.Cu") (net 12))
 (segment (start 106.15 50.775) (end 105.975 50.95) (width 0.25) (layer "F.Cu") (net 12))
 (segment (start 108.33 50.775) (end 106.15 50.775) (width 0.25) (layer "F.Cu") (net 12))
 (segment (start 105.975 52.825) (end 107.3 54.15) (width 0.25) (layer "F.Cu") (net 12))
 (segment (start 113.085 46.02) (end 108.33 50.775) (width 0.25) (layer "F.Cu") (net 12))
 (segment (start 113.085 44.945) (end 113.085 46.02) (width 0.25) (layer "F.Cu") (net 12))
 (segment (start 128.35 118.85) (end 121.85 118.85) (width 0.25) (layer "F.Cu") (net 19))
 (segment (start 101.95 118.9) (end 108.45 118.9) (width 0.25) (layer "F.Cu") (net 19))
 (segment (start 128.35 118.85) (end 128.35 121.06) (width 0.25) (layer "F.Cu") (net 19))
 (segment (start 118.35 118.9) (end 111.85 118.9) (width 0.25) (layer "F.Cu") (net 19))
 (segment (start 128.35 118.85) (end 131.6 118.85) (width 0.25) (layer "F.Cu") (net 19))
 (segment (start 121.303899 128.106101) (end 114.342499 128.106101) (width 0.25) (layer "F.Cu") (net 19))
 (segment (start 108.45 118.9) (end 111.85 118.9) (width 0.25) (layer "F.Cu") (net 19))
 (segment (start 122.7575 126.6525) (end 121.303899 128.106101) (width 0.25) (layer "F.Cu") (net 19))
 (segment (start 128.35 121.06) (end 122.7575 126.6525) (width 0.25) (layer "F.Cu") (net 19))
 (segment (start 111.85 125.613602) (end 111.85 118.9) (width 0.25) (layer "F.Cu") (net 19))
 (segment (start 114.342499 128.106101) (end 111.85 125.613602) (width 0.25) (layer "F.Cu") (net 19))
 (segment (start 138.15 118.9) (end 131.65 118.9) (width 0.25) (layer "F.Cu") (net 19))
 (segment (start 131.6 118.85) (end 131.65 118.9) (width 0.25) (layer "F.Cu") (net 19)))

